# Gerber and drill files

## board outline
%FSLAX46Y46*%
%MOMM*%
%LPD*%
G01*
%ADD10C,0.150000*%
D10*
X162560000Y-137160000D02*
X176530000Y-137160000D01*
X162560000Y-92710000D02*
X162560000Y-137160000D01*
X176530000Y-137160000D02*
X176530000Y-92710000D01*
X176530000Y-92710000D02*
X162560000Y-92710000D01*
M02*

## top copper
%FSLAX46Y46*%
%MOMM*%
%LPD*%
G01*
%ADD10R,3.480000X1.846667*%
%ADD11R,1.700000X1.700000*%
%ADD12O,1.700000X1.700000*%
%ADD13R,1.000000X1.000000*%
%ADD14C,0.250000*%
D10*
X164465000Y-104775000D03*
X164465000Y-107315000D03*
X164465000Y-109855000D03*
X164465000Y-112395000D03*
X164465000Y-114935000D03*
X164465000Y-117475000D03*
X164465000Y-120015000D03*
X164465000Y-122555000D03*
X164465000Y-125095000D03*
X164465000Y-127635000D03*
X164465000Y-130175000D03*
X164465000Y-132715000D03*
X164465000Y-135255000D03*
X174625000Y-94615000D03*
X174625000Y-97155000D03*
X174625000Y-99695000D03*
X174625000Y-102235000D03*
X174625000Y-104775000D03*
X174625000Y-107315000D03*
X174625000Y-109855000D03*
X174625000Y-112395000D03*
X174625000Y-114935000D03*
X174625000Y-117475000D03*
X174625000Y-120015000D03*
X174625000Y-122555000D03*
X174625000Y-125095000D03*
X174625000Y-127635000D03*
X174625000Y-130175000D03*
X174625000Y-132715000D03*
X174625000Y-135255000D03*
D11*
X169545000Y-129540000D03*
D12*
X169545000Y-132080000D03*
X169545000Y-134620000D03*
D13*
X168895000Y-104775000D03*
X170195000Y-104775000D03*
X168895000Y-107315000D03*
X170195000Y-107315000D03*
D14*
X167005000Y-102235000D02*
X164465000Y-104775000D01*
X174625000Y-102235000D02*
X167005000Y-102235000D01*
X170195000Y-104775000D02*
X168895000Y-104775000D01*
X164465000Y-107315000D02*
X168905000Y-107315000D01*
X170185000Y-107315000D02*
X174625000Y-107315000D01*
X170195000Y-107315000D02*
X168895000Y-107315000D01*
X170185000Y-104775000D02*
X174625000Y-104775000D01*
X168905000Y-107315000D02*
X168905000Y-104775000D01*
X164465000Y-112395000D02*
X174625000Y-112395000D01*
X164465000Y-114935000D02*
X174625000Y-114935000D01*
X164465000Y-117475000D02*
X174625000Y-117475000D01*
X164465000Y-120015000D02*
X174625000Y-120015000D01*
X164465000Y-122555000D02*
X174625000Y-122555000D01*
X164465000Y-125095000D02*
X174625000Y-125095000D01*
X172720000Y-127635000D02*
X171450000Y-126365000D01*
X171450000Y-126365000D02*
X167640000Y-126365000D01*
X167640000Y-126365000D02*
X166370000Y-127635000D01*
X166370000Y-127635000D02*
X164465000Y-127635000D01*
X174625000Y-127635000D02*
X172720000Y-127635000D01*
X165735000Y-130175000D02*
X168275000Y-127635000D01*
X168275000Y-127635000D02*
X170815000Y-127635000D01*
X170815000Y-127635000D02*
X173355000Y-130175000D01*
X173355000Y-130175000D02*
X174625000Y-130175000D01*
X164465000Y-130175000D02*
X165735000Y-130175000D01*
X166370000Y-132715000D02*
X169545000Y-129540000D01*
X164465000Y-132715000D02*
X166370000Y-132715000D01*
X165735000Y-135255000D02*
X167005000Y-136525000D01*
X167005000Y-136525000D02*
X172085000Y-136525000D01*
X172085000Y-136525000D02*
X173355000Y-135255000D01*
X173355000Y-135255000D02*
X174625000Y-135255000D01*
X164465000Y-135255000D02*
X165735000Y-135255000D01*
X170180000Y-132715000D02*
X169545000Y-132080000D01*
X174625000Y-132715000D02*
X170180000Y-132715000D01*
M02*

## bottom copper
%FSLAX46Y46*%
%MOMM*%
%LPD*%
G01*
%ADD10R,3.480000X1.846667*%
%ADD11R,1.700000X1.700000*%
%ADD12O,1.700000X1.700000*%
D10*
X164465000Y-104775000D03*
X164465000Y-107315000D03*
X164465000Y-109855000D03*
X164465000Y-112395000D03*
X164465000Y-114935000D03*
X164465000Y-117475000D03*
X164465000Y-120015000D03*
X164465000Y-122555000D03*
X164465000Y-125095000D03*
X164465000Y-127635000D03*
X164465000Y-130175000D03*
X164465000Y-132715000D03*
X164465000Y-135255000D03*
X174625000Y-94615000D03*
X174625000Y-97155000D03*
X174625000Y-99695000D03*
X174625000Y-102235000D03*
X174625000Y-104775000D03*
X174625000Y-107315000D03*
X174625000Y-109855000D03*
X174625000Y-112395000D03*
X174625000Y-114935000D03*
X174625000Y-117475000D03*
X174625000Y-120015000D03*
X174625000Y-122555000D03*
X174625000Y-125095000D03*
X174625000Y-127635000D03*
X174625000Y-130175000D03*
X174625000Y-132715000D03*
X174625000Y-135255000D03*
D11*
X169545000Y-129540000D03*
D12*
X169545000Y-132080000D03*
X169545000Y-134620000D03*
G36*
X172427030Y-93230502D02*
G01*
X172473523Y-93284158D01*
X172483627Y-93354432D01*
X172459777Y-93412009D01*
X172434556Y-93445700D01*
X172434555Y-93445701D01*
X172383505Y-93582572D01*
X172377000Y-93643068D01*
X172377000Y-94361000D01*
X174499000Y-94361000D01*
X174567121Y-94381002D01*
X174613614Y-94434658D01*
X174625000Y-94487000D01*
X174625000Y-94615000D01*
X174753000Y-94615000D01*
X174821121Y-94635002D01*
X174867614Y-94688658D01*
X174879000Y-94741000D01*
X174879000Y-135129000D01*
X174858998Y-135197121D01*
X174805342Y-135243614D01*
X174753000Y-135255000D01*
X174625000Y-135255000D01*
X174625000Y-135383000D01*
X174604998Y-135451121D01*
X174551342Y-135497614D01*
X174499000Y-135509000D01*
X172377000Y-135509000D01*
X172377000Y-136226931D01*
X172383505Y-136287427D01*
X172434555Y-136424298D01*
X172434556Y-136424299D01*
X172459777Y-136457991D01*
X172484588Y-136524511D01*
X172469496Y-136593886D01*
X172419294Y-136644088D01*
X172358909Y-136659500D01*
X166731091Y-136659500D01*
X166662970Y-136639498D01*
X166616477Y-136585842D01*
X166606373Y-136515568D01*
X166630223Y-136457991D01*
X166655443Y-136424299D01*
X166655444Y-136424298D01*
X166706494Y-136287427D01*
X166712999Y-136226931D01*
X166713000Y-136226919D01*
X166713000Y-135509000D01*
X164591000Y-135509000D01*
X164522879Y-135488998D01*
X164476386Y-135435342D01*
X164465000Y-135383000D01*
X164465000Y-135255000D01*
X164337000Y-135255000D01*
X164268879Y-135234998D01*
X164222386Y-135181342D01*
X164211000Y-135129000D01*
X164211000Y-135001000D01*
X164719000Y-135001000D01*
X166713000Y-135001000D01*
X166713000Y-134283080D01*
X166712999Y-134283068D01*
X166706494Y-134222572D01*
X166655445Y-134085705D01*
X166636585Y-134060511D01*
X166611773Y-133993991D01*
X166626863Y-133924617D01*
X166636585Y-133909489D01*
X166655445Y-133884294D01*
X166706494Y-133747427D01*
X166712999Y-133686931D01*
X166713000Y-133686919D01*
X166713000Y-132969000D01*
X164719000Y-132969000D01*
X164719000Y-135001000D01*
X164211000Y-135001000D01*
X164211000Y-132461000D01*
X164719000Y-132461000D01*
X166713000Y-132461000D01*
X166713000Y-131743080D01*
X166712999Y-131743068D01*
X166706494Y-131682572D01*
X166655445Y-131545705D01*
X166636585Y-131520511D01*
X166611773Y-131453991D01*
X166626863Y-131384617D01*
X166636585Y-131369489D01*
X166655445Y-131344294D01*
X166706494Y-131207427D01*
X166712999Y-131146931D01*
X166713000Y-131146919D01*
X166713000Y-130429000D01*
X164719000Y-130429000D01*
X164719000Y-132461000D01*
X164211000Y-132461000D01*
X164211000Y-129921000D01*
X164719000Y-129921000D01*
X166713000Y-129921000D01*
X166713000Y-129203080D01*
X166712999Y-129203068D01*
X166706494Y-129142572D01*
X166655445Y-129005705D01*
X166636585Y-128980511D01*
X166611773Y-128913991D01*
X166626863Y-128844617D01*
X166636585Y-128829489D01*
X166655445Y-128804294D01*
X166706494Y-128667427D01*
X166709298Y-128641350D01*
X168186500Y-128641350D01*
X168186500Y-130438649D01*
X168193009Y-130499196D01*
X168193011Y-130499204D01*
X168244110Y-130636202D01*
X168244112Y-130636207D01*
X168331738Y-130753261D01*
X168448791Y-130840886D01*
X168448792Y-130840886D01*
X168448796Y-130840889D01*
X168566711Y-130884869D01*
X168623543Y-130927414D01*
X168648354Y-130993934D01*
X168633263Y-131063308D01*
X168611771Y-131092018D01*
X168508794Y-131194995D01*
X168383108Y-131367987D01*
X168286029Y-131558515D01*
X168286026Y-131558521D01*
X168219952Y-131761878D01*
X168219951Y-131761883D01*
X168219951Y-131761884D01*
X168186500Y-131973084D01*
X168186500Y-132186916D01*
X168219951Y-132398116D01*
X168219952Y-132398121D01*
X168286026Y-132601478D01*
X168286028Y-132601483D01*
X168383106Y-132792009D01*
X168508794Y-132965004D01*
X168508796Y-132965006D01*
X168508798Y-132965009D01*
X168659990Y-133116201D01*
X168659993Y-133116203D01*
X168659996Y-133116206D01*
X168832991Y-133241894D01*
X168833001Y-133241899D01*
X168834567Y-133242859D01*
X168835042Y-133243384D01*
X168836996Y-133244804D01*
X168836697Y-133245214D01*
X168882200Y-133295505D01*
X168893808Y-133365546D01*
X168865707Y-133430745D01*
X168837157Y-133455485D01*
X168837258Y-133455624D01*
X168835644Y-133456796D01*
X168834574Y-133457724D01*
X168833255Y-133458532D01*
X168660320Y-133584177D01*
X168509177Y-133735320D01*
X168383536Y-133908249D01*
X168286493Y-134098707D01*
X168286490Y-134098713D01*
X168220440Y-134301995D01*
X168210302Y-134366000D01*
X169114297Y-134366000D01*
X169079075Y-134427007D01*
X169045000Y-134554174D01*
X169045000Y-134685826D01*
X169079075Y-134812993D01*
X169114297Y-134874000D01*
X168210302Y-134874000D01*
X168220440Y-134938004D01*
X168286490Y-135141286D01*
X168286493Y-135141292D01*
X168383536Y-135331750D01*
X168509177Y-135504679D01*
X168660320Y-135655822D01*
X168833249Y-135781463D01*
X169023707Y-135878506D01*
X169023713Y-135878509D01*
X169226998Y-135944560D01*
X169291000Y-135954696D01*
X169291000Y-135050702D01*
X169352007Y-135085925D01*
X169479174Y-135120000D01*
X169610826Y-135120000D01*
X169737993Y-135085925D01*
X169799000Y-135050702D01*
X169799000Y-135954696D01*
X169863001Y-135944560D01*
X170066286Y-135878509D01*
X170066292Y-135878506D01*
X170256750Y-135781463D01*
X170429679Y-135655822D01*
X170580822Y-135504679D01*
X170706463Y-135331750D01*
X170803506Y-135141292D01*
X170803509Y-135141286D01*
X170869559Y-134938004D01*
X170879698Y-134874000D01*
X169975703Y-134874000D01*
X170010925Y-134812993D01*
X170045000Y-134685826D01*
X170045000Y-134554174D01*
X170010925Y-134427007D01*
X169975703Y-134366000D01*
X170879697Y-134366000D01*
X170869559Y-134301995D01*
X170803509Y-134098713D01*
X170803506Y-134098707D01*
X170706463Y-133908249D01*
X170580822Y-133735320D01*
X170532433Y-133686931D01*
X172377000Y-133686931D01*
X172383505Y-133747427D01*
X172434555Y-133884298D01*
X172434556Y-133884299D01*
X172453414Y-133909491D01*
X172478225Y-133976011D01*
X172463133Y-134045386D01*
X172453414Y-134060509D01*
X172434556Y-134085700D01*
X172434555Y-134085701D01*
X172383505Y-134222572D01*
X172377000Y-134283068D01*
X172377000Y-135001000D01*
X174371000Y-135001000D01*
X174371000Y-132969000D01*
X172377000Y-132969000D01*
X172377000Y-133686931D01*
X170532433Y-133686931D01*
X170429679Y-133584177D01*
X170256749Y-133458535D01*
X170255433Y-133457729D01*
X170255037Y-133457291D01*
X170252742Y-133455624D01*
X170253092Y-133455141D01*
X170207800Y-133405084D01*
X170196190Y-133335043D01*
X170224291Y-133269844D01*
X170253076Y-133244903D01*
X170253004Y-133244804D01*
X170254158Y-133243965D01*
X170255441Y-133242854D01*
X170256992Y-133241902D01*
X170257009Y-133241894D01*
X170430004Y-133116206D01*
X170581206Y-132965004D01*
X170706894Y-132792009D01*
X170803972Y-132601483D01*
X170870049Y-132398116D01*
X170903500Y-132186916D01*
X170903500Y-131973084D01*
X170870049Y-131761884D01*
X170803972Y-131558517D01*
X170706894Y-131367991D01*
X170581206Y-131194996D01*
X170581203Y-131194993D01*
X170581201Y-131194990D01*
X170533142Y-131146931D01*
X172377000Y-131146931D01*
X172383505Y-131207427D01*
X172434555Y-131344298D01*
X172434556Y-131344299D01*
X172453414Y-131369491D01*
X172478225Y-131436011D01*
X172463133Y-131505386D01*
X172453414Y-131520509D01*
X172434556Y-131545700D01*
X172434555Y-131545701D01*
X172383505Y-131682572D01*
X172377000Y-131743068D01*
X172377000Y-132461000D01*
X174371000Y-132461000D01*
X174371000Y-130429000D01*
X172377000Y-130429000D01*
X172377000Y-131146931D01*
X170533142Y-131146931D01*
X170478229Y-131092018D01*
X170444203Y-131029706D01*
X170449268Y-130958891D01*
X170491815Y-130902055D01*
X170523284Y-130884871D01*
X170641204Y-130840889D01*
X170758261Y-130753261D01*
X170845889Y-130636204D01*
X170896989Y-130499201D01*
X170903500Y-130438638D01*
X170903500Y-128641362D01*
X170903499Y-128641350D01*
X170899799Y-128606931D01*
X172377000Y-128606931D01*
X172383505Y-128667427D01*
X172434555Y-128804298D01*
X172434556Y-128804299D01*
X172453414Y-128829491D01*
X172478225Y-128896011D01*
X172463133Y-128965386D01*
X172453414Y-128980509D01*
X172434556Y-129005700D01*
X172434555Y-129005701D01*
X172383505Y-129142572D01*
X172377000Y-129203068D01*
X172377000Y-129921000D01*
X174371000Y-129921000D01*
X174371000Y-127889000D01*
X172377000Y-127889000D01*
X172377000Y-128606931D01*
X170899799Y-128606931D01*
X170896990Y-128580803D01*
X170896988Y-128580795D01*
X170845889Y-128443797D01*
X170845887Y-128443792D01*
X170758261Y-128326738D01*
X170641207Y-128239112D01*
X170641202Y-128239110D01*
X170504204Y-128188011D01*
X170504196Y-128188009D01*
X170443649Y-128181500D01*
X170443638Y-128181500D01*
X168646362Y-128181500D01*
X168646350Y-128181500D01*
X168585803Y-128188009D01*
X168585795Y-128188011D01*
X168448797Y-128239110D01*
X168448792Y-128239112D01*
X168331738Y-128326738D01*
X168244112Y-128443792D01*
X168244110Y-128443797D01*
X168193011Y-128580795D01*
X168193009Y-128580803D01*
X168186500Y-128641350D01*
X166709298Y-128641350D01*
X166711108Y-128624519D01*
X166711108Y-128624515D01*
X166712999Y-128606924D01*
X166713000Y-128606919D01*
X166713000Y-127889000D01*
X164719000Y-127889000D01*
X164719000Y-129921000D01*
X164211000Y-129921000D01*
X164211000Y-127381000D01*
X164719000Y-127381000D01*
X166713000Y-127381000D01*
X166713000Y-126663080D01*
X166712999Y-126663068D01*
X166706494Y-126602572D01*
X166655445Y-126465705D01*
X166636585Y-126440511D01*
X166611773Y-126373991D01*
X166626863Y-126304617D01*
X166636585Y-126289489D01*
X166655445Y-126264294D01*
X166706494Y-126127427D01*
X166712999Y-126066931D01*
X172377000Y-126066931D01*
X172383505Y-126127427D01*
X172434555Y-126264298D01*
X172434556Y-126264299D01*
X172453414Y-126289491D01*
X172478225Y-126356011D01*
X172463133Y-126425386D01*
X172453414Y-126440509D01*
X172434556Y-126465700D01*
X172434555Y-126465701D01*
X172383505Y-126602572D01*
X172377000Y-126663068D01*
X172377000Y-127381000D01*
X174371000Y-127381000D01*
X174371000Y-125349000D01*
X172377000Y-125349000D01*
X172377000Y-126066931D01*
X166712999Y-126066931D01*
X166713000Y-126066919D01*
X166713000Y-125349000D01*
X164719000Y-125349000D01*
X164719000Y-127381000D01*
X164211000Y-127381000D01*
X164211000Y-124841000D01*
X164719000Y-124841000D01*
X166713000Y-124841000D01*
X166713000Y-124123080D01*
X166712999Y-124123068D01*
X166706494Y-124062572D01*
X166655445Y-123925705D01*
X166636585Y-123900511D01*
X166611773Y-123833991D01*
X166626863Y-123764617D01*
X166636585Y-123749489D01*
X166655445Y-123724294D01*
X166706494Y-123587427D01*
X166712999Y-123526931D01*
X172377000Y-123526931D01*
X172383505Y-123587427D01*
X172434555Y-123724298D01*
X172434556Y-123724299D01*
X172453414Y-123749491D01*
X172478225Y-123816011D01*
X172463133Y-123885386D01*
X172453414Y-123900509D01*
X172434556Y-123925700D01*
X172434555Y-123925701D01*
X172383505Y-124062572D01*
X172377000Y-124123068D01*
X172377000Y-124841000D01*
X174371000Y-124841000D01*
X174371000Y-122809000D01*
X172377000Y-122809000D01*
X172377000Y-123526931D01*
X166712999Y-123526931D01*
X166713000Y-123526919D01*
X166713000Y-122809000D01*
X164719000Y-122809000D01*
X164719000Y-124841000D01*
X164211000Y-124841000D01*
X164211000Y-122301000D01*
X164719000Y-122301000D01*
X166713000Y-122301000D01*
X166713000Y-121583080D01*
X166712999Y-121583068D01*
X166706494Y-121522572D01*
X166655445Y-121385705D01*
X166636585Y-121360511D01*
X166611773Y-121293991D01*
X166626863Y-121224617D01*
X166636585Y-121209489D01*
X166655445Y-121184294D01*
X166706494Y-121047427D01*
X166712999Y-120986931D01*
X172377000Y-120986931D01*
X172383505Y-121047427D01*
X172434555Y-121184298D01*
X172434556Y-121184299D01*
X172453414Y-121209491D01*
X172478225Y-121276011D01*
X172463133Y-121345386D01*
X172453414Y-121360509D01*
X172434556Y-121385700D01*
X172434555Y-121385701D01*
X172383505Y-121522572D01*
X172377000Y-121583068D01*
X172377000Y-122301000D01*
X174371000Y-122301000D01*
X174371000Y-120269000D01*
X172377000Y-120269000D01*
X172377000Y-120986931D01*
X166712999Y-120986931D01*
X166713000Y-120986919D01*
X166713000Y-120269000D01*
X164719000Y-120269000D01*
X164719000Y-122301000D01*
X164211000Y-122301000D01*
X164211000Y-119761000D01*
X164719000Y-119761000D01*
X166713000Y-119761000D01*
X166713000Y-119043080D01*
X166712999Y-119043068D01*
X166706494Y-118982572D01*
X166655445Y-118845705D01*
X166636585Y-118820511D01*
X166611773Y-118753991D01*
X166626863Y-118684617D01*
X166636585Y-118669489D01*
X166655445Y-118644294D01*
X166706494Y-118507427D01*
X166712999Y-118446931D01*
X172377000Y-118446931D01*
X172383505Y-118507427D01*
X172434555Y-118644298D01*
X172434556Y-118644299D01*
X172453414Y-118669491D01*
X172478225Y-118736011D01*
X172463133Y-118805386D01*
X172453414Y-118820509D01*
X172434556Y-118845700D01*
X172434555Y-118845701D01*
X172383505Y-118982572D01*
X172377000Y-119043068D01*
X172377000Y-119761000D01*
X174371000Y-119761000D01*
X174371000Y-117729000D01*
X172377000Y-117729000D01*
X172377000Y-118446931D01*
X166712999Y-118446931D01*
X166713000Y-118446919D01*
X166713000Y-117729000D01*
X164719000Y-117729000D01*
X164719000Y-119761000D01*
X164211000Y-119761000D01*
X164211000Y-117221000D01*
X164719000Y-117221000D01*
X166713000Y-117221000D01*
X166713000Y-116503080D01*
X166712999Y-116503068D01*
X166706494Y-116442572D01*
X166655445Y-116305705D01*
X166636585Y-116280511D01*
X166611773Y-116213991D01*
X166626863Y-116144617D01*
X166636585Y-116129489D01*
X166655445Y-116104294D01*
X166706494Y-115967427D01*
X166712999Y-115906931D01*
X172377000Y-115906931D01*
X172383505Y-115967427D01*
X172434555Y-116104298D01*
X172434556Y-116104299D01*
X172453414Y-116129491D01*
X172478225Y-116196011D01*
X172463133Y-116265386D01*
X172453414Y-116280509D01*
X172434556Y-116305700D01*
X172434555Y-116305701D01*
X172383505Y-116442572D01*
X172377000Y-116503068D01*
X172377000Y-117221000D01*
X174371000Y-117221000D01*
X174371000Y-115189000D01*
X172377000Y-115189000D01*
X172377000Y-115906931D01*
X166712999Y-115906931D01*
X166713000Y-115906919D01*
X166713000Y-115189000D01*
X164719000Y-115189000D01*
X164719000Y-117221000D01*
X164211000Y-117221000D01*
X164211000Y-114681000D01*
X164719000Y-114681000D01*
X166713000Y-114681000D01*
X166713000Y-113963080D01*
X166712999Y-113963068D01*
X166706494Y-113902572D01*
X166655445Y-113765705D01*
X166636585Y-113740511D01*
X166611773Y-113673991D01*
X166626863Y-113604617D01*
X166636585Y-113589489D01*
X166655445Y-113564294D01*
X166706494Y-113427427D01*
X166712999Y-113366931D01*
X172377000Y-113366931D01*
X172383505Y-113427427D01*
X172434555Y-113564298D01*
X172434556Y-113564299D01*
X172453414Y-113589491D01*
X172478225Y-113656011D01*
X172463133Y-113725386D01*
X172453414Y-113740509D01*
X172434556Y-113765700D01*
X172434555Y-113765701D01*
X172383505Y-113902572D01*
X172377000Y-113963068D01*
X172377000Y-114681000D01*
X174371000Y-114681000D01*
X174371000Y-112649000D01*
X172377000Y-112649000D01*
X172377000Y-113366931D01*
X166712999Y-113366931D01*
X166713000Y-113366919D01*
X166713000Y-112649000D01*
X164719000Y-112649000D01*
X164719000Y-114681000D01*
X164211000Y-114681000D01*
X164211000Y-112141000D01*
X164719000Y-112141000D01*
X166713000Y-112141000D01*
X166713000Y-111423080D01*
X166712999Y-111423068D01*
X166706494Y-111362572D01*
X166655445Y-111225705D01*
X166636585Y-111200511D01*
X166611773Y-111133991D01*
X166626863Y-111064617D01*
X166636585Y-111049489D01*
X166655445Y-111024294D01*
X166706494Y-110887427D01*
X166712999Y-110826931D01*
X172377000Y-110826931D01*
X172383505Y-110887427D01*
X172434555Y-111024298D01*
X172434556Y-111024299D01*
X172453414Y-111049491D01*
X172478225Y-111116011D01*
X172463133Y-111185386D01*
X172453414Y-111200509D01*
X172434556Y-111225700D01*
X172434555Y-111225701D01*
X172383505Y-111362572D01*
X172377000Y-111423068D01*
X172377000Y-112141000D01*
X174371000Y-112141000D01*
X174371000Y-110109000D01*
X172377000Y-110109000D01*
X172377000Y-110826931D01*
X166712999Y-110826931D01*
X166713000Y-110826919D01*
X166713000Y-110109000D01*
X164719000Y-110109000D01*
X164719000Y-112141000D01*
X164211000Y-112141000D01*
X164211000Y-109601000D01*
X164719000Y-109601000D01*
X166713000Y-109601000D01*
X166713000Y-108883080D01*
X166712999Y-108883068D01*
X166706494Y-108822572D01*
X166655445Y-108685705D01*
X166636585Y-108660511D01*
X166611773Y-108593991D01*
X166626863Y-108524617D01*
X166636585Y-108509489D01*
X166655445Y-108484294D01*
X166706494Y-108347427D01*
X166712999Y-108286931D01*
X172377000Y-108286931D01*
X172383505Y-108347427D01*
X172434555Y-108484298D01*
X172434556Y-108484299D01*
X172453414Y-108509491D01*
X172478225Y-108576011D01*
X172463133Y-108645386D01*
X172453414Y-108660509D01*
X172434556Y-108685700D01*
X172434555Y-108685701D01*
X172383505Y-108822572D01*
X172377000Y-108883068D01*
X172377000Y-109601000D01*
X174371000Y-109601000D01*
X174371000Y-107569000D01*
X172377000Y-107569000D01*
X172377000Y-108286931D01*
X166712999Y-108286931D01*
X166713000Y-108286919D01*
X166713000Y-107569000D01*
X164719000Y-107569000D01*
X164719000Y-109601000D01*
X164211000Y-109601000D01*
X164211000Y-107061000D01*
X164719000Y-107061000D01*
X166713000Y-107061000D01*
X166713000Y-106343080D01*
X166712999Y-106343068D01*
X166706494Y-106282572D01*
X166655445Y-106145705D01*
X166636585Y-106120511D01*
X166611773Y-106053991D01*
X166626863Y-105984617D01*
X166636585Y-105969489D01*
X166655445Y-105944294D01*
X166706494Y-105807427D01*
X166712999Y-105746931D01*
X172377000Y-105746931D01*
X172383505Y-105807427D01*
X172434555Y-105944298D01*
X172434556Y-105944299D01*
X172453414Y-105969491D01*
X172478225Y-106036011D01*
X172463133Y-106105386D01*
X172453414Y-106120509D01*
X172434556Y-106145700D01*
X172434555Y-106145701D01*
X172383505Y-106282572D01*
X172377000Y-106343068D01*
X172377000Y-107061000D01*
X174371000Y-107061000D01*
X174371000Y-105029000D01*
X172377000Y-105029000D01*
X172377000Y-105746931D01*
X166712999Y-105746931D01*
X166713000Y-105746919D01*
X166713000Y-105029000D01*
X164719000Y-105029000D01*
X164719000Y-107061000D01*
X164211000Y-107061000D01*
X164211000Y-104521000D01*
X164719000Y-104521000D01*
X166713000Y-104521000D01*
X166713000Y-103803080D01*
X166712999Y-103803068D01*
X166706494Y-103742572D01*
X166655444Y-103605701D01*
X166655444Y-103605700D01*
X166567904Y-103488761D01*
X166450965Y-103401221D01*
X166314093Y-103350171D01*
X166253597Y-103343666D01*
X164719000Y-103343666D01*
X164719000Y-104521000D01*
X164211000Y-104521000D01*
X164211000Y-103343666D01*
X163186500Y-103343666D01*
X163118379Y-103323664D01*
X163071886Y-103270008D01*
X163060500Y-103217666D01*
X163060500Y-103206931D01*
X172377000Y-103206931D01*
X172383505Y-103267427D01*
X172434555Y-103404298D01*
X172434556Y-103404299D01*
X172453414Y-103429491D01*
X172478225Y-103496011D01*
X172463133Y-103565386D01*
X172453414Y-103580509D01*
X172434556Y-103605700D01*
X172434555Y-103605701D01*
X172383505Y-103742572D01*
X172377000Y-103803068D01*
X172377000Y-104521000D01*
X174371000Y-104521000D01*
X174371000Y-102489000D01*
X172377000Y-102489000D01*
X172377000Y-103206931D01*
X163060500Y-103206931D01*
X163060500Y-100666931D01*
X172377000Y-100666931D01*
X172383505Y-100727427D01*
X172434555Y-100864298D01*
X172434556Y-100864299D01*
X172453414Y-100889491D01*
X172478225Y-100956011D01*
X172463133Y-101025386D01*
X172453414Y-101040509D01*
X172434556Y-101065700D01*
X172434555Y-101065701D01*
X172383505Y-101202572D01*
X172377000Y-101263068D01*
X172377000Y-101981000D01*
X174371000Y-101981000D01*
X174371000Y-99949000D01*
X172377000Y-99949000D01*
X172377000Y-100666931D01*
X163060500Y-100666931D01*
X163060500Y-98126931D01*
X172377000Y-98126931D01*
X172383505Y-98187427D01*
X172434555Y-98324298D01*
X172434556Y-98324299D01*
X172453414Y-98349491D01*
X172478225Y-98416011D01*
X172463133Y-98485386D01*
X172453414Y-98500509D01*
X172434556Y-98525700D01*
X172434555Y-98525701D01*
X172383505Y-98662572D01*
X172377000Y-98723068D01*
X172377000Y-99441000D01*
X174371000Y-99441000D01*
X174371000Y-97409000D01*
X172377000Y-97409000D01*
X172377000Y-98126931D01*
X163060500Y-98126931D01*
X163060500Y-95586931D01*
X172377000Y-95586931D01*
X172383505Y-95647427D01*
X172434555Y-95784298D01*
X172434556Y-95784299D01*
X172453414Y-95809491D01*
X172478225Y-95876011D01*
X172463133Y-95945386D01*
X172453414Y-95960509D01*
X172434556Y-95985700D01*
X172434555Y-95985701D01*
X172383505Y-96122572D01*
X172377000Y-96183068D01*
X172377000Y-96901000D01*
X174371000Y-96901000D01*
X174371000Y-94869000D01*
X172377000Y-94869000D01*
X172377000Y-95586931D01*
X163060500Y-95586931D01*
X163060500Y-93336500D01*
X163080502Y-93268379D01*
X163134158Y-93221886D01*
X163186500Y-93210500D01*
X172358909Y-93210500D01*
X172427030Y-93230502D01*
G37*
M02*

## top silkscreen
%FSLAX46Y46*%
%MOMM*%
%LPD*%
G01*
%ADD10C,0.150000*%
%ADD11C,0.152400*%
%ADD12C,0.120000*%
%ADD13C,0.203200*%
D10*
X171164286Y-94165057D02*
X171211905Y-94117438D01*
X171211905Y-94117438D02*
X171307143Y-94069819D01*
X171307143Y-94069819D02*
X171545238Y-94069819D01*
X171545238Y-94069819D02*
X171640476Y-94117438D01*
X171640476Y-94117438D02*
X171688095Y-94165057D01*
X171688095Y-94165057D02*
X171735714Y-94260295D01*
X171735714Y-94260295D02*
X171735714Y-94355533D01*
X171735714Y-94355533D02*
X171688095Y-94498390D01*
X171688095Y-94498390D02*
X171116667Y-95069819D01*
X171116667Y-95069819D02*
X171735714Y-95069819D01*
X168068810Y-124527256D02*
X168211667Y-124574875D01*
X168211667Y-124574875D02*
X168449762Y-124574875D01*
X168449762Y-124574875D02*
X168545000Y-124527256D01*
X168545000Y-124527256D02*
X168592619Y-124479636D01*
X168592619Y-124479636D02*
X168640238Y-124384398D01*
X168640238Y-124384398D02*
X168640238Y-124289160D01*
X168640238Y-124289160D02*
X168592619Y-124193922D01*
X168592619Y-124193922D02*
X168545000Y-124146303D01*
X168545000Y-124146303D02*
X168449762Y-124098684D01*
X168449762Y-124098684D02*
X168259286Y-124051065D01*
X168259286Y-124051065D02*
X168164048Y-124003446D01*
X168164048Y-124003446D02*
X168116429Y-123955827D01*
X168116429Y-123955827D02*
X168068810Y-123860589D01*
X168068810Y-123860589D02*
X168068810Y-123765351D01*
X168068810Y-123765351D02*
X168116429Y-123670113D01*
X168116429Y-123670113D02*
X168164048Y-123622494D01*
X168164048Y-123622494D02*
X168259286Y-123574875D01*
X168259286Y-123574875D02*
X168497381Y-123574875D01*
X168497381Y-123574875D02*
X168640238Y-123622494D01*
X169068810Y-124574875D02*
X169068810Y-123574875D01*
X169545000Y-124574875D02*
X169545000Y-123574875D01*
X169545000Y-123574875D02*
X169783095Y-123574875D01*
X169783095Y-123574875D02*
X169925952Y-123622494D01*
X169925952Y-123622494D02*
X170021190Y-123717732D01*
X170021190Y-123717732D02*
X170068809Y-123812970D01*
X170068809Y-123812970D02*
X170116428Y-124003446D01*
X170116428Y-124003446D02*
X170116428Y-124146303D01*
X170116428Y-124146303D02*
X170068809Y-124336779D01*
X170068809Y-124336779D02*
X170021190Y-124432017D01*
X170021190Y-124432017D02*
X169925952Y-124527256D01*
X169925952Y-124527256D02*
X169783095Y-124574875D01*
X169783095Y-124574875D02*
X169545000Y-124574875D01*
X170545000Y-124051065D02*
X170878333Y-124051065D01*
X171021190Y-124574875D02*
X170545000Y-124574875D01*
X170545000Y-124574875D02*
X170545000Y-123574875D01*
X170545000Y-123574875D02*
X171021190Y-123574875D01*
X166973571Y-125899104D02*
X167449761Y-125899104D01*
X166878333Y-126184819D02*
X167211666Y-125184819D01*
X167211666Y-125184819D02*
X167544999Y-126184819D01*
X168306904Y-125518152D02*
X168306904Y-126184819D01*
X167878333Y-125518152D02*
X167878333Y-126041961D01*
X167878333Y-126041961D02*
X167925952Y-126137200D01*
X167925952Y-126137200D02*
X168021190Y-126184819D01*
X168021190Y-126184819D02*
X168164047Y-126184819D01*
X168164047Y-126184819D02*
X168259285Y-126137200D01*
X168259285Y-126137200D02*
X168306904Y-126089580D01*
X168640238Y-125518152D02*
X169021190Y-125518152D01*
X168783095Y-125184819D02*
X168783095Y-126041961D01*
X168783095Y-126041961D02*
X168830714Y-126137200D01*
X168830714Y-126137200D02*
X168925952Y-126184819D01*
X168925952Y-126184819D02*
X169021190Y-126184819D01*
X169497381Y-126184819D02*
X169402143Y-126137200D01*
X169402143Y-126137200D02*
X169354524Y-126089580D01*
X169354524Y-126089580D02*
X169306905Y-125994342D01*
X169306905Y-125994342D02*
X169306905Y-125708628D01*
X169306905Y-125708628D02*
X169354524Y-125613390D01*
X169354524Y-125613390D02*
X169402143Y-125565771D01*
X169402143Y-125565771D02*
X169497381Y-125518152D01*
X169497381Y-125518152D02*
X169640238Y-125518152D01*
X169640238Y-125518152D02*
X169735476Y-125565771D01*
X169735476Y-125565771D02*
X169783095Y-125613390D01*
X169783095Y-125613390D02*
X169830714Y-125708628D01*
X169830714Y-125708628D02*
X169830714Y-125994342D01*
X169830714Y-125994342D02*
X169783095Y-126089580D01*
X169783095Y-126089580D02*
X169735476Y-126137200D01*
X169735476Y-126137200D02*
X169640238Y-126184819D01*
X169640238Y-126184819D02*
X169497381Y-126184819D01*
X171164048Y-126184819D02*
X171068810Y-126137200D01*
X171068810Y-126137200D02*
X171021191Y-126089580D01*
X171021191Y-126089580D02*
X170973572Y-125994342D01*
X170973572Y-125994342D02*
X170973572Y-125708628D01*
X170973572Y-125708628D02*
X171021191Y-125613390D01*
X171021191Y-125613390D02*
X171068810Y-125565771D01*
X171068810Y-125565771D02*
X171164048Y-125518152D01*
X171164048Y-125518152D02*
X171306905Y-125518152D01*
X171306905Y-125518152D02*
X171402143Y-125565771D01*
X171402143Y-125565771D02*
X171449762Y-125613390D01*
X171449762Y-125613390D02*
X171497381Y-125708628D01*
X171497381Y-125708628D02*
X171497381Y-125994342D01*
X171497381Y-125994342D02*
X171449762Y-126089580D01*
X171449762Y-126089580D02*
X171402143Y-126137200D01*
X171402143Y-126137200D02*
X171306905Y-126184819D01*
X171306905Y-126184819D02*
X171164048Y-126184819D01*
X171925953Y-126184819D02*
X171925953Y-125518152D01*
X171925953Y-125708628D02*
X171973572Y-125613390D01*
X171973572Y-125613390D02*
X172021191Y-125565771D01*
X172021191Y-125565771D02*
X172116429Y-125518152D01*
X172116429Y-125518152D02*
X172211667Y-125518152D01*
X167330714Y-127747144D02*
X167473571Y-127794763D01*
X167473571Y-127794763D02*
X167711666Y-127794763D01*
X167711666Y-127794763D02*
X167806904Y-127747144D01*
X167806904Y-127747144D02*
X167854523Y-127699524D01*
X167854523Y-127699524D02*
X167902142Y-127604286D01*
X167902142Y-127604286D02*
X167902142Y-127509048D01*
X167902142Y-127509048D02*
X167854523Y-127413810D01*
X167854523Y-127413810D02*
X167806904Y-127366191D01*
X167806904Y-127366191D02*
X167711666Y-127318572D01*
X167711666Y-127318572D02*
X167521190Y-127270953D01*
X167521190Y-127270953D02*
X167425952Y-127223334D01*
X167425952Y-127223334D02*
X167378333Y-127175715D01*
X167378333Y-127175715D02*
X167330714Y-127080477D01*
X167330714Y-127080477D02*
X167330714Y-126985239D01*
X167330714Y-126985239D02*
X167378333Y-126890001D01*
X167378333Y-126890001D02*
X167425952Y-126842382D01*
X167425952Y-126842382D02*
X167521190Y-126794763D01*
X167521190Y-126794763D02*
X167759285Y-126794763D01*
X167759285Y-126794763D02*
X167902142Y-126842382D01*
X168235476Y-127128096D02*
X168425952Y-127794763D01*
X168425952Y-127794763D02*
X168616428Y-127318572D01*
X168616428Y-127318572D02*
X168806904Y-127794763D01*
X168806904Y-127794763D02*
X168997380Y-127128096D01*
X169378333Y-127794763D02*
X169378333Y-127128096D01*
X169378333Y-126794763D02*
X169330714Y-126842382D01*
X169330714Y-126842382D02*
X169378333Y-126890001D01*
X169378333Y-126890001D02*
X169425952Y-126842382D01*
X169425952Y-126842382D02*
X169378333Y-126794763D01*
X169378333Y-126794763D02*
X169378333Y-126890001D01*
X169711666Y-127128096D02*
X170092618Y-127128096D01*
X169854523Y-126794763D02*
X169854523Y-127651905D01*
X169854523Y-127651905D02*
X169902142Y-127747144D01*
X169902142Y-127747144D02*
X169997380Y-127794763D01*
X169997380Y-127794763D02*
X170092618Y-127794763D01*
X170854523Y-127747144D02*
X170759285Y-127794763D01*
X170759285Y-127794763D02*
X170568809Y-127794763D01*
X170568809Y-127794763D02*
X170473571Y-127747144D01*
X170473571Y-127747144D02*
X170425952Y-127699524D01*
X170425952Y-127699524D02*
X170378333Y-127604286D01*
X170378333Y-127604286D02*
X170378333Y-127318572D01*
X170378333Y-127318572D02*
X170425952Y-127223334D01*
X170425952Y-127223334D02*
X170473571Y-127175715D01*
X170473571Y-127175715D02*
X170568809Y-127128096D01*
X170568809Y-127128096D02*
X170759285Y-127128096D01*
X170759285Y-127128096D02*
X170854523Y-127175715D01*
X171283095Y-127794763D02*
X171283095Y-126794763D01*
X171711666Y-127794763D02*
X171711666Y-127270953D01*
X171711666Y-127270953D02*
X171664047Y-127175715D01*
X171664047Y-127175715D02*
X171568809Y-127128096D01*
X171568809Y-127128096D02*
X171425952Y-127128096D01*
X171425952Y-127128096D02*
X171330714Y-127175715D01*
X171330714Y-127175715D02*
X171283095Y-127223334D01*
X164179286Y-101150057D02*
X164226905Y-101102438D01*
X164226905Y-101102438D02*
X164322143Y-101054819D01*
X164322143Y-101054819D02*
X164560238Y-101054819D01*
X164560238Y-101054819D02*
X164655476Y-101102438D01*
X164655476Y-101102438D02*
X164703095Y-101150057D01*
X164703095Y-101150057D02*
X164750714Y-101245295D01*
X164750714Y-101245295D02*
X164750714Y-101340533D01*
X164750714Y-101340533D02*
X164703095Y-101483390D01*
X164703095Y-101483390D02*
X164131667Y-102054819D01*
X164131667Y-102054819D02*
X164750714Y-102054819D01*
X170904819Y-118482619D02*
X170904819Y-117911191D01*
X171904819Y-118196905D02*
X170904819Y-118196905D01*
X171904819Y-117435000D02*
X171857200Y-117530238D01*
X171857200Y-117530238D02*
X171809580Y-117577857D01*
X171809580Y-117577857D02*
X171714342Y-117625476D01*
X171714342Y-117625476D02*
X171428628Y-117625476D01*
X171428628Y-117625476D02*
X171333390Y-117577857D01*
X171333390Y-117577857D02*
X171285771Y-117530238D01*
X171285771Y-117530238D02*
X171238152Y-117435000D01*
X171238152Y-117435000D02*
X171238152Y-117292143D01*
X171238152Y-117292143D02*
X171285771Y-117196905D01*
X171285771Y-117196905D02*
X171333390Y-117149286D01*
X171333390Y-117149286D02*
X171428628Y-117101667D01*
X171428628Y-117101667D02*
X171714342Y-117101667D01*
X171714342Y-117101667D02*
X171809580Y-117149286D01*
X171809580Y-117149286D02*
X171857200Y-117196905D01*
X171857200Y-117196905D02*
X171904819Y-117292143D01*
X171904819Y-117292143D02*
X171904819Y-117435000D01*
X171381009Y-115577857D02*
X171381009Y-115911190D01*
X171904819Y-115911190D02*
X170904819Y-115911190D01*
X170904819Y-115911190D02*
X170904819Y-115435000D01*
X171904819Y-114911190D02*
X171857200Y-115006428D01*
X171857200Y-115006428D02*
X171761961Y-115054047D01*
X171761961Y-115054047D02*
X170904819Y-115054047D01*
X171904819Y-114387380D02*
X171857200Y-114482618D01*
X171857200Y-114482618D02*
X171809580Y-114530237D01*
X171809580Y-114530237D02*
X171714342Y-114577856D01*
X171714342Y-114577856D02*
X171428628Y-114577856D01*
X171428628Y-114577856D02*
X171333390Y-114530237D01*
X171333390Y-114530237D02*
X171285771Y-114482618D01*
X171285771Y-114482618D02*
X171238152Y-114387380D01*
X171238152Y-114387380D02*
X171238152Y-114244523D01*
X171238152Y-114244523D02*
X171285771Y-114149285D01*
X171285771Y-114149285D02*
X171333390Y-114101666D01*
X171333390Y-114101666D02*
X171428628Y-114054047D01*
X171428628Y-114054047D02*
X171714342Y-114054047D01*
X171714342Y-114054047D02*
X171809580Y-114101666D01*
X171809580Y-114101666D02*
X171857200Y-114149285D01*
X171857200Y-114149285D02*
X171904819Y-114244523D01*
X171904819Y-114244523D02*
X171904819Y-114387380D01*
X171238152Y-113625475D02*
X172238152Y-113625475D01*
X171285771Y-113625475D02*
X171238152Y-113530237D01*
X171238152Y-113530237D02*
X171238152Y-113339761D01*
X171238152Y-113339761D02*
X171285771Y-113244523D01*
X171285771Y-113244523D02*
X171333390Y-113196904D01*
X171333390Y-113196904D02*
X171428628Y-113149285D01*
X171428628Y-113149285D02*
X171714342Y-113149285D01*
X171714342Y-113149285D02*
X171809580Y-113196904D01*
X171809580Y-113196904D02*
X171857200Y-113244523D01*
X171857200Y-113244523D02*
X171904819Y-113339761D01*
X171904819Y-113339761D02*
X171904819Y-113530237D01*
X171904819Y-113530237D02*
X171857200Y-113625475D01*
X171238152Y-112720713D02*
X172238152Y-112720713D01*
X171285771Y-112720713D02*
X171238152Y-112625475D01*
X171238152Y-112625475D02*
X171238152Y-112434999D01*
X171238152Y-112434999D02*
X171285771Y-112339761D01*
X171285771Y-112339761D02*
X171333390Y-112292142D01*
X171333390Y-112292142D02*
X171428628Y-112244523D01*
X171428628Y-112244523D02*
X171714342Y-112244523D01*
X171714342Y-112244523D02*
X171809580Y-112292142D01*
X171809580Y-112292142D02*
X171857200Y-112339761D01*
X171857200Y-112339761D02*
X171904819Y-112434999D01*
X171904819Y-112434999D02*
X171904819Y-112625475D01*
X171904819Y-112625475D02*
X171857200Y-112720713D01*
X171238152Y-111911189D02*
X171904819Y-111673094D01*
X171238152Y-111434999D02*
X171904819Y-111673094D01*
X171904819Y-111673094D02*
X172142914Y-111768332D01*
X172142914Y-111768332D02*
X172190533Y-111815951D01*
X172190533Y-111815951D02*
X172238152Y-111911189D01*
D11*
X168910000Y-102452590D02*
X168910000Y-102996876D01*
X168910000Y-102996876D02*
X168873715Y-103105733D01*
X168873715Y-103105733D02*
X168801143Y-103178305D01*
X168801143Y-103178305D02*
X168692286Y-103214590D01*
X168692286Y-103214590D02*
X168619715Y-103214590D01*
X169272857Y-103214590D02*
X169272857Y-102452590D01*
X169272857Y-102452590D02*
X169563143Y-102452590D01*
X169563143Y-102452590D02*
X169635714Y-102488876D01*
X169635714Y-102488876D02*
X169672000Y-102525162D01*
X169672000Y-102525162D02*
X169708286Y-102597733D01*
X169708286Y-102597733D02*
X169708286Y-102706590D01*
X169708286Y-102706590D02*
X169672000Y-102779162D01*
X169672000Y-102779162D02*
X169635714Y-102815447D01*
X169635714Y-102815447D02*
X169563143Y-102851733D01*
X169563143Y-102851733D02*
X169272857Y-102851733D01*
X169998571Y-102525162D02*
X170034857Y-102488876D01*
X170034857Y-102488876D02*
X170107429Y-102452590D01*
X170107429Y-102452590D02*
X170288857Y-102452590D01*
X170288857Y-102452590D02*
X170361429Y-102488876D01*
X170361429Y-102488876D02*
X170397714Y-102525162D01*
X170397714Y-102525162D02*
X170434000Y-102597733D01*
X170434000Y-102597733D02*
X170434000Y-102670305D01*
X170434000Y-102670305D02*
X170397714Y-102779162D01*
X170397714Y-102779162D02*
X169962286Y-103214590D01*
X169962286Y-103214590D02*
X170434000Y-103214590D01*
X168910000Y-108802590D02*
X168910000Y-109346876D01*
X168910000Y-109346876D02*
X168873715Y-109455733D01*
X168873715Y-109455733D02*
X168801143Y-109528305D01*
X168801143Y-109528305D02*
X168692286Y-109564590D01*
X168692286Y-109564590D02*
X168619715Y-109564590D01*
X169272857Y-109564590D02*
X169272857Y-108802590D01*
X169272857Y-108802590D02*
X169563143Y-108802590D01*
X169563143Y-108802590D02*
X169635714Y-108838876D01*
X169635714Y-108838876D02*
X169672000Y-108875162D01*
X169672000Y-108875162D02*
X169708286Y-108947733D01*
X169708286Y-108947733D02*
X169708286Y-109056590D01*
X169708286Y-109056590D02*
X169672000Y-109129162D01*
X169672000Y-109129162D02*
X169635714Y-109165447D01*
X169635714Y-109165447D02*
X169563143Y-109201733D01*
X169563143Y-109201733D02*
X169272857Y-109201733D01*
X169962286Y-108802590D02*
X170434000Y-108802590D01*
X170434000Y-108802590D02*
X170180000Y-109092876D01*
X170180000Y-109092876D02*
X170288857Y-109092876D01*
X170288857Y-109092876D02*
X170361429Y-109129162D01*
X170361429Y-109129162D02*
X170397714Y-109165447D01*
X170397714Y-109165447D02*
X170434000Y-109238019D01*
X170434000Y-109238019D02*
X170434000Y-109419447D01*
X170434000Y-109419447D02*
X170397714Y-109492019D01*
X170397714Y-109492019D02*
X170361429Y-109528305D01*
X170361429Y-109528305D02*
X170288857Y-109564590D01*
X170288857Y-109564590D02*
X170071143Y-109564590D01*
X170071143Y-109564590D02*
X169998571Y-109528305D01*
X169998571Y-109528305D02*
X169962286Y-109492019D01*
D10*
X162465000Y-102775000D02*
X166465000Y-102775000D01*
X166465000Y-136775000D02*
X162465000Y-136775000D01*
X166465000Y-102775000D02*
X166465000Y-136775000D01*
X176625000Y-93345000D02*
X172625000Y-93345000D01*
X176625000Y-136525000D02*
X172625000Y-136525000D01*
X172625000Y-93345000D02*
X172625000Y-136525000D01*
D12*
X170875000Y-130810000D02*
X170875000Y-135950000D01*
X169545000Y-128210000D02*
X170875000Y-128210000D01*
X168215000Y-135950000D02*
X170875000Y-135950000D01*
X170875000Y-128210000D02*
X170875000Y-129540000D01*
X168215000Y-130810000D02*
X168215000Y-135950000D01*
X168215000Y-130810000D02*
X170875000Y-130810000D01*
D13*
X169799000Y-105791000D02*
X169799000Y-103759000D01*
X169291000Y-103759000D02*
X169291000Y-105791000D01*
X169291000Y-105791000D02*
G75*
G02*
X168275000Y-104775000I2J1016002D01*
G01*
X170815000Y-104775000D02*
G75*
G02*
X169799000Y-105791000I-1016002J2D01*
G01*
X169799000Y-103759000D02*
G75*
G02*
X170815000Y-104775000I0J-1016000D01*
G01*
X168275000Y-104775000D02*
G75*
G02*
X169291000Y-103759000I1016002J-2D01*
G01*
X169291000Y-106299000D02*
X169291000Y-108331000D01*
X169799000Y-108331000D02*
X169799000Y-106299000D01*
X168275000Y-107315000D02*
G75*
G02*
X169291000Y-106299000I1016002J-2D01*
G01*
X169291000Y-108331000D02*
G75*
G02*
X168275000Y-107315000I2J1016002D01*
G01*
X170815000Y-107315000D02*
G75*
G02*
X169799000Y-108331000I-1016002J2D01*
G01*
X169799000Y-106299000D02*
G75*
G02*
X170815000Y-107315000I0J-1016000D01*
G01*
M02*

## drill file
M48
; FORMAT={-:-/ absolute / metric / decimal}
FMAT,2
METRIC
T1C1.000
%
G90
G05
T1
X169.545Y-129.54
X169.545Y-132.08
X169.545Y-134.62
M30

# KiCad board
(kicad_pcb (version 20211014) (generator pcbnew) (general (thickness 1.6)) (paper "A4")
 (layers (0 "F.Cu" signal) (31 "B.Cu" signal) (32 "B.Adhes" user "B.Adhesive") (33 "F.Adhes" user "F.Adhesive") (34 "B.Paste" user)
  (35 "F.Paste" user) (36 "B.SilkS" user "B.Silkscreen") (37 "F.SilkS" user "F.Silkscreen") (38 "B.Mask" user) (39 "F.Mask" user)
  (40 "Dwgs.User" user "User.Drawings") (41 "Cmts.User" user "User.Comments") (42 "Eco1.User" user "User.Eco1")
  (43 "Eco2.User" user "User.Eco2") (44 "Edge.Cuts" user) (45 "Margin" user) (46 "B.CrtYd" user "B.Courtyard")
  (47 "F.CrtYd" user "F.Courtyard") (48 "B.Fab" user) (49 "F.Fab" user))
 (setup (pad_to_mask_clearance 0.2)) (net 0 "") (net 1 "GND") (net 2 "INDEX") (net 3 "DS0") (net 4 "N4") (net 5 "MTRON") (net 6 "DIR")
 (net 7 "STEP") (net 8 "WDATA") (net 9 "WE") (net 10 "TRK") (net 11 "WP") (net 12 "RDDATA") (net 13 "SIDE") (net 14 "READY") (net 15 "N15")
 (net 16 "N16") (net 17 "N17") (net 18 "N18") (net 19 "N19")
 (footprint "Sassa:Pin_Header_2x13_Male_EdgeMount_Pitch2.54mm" (layer "F.Cu") (at 164.465 104.775 -90)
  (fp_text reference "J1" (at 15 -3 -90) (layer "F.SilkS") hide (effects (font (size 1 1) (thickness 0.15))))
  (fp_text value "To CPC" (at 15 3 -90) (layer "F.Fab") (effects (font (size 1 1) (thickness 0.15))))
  (fp_line (start -2 2) (end -2 -2) (layer "F.SilkS") (width 0.15))
  (fp_line (start 32 -2) (end 32 2) (layer "F.SilkS") (width 0.15))
  (fp_line (start -2 -2) (end 32 -2) (layer "F.SilkS") (width 0.15))
  (pad "1" smd rect locked (at 0 0 270) (size 1.846667 3.48) (layers "B.Cu" "B.Paste" "B.Mask") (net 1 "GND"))
  (pad "2" smd rect locked (at 0 0 270) (size 1.846667 3.48) (layers "F.Cu" "F.Paste" "F.Mask") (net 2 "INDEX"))
  (pad "3" smd rect locked (at 2.54 0 270) (size 1.846667 3.48) (layers "B.Cu" "B.Paste" "B.Mask") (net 1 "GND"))
  (pad "4" smd rect locked (at 2.54 0 270) (size 1.846667 3.48) (layers "F.Cu" "F.Paste" "F.Mask") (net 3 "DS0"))
  (pad "5" smd rect locked (at 5.08 0 270) (size 1.846667 3.48) (layers "B.Cu" "B.Paste" "B.Mask") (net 1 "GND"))
  (pad "6" smd rect locked (at 5.08 0 270) (size 1.846667 3.48) (layers "F.Cu" "F.Paste" "F.Mask") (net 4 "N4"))
  (pad "7" smd rect locked (at 7.62 0 270) (size 1.846667 3.48) (layers "B.Cu" "B.Paste" "B.Mask") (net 1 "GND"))
  (pad "8" smd rect locked (at 7.62 0 270) (size 1.846667 3.48) (layers "F.Cu" "F.Paste" "F.Mask") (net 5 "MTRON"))
  (pad "9" smd rect locked (at 10.16 0 270) (size 1.846667 3.48) (layers "B.Cu" "B.Paste" "B.Mask") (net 1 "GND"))
  (pad "10" smd rect locked (at 10.16 0 270) (size 1.846667 3.48) (layers "F.Cu" "F.Paste" "F.Mask") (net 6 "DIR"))
  (pad "11" smd rect locked (at 12.7 0 270) (size 1.846667 3.48) (layers "B.Cu" "B.Paste" "B.Mask") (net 1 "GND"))
  (pad "12" smd rect locked (at 12.7 0 270) (size 1.846667 3.48) (layers "F.Cu" "F.Paste" "F.Mask") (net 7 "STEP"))
  (pad "13" smd rect locked (at 15.24 0 270) (size 1.846667 3.48) (layers "B.Cu" "B.Paste" "B.Mask") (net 1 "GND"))
  (pad "14" smd rect locked (at 15.24 0 270) (size 1.846667 3.48) (layers "F.Cu" "F.Paste" "F.Mask") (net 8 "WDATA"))
  (pad "15" smd rect locked (at 17.78 0 270) (size 1.846667 3.48) (layers "B.Cu" "B.Paste" "B.Mask") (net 1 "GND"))
  (pad "16" smd rect locked (at 17.78 0 270) (size 1.846667 3.48) (layers "F.Cu" "F.Paste" "F.Mask") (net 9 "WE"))
  (pad "17" smd rect locked (at 20.32 0 270) (size 1.846667 3.48) (layers "B.Cu" "B.Paste" "B.Mask") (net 1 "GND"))
  (pad "18" smd rect locked (at 20.32 0 270) (size 1.846667 3.48) (layers "F.Cu" "F.Paste" "F.Mask") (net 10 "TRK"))
  (pad "19" smd rect locked (at 22.86 0 270) (size 1.846667 3.48) (layers "B.Cu" "B.Paste" "B.Mask") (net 1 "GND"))
  (pad "20" smd rect locked (at 22.86 0 270) (size 1.846667 3.48) (layers "F.Cu" "F.Paste" "F.Mask") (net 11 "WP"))
  (pad "21" smd rect locked (at 25.4 0 270) (size 1.846667 3.48) (layers "B.Cu" "B.Paste" "B.Mask") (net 1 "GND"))
  (pad "22" smd rect locked (at 25.4 0 270) (size 1.846667 3.48) (layers "F.Cu" "F.Paste" "F.Mask") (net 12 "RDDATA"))
  (pad "23" smd rect locked (at 27.94 0 270) (size 1.846667 3.48) (layers "B.Cu" "B.Paste" "B.Mask") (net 1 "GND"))
  (pad "24" smd rect locked (at 27.94 0 270) (size 1.846667 3.48) (layers "F.Cu" "F.Paste" "F.Mask") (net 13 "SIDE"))
  (pad "25" smd rect locked (at 30.48 0 270) (size 1.846667 3.48) (layers "B.Cu" "B.Paste" "B.Mask") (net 1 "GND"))
  (pad "26" smd rect locked (at 30.48 0 270) (size 1.846667 3.48) (layers "F.Cu" "F.Paste" "F.Mask") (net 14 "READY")))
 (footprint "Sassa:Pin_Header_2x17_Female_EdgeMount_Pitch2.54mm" (layer "F.Cu") (at 174.625 135.255 90)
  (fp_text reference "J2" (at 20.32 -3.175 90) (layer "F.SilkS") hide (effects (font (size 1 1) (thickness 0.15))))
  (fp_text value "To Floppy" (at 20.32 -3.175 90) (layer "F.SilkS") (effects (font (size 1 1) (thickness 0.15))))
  (fp_line (start 41.91 2) (end 41.91 -2) (layer "F.SilkS") (width 0.15))
  (fp_line (start -1.27 2) (end -1.27 -2) (layer "F.SilkS") (width 0.15))
  (fp_line (start 41.91 -2) (end -1.27 -2) (layer "F.SilkS") (width 0.15))
  (pad "1" smd rect (at 40.64 0 90) (size 1.846667 3.48) (layers "B.Cu" "B.Paste" "B.Mask") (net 1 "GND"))
  (pad "2" smd rect (at 40.64 0 90) (size 1.846667 3.48) (layers "F.Cu" "F.Paste" "F.Mask") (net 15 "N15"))
  (pad "3" smd rect (at 38.1 0 90) (size 1.846667 3.48) (layers "B.Cu" "B.Paste" "B.Mask") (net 1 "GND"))
  (pad "4" smd rect (at 38.1 0 90) (size 1.846667 3.48) (layers "F.Cu" "F.Paste" "F.Mask") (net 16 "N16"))
  (pad "5" smd rect (at 35.56 0 90) (size 1.846667 3.48) (layers "B.Cu" "B.Paste" "B.Mask") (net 1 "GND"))
  (pad "6" smd rect (at 35.56 0 90) (size 1.846667 3.48) (layers "F.Cu" "F.Paste" "F.Mask") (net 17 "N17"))
  (pad "7" smd rect (at 33.02 0 90) (size 1.846667 3.48) (layers "B.Cu" "B.Paste" "B.Mask") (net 1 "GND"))
  (pad "8" smd rect (at 33.02 0 90) (size 1.846667 3.48) (layers "F.Cu" "F.Paste" "F.Mask") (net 2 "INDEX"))
  (pad "9" smd rect (at 30.48 0 90) (size 1.846667 3.48) (layers "B.Cu" "B.Paste" "B.Mask") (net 1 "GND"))
  (pad "10" smd rect (at 30.48 0 90) (size 1.846667 3.48) (layers "F.Cu" "F.Paste" "F.Mask") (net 3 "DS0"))
  (pad "11" smd rect (at 27.94 0 90) (size 1.846667 3.48) (layers "B.Cu" "B.Paste" "B.Mask") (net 1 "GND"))
  (pad "12" smd rect (at 27.94 0 90) (size 1.846667 3.48) (layers "F.Cu" "F.Paste" "F.Mask") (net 3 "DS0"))
  (pad "13" smd rect (at 25.4 0 90) (size 1.846667 3.48) (layers "B.Cu" "B.Paste" "B.Mask") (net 1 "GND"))
  (pad "14" smd rect (at 25.4 0 90) (size 1.846667 3.48) (layers "F.Cu" "F.Paste" "F.Mask") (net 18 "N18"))
  (pad "15" smd rect (at 22.86 0 90) (size 1.846667 3.48) (layers "B.Cu" "B.Paste" "B.Mask") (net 1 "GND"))
  (pad "16" smd rect (at 22.86 0 90) (size 1.846667 3.48) (layers "F.Cu" "F.Paste" "F.Mask") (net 5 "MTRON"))
  (pad "17" smd rect (at 20.32 0 90) (size 1.846667 3.48) (layers "B.Cu" "B.Paste" "B.Mask") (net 1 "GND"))
  (pad "18" smd rect (at 20.32 0 90) (size 1.846667 3.48) (layers "F.Cu" "F.Paste" "F.Mask") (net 6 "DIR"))
  (pad "19" smd rect (at 17.78 0 90) (size 1.846667 3.48) (layers "B.Cu" "B.Paste" "B.Mask") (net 1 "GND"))
  (pad "20" smd rect (at 17.78 0 90) (size 1.846667 3.48) (layers "F.Cu" "F.Paste" "F.Mask") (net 7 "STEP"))
  (pad "21" smd rect (at 15.24 0 90) (size 1.846667 3.48) (layers "B.Cu" "B.Paste" "B.Mask") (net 1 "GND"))
  (pad "22" smd rect (at 15.24 0 90) (size 1.846667 3.48) (layers "F.Cu" "F.Paste" "F.Mask") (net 8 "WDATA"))
  (pad "23" smd rect (at 12.7 0 90) (size 1.846667 3.48) (layers "B.Cu" "B.Paste" "B.Mask") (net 1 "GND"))
  (pad "24" smd rect (at 12.7 0 90) (size 1.846667 3.48) (layers "F.Cu" "F.Paste" "F.Mask") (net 9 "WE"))
  (pad "25" smd rect (at 10.16 0 90) (size 1.846667 3.48) (layers "B.Cu" "B.Paste" "B.Mask") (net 1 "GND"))
  (pad "26" smd rect (at 10.16 0 90) (size 1.846667 3.48) (layers "F.Cu" "F.Paste" "F.Mask") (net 10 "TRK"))
  (pad "27" smd rect (at 7.62 0 90) (size 1.846667 3.48) (layers "B.Cu" "B.Paste" "B.Mask") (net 1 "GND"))
  (pad "28" smd rect (at 7.62 0 90) (size 1.846667 3.48) (layers "F.Cu" "F.Paste" "F.Mask") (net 11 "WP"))
  (pad "29" smd rect (at 5.08 0 90) (size 1.846667 3.48) (layers "B.Cu" "B.Paste" "B.Mask") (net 1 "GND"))
  (pad "30" smd rect (at 5.08 0 90) (size 1.846667 3.48) (layers "F.Cu" "F.Paste" "F.Mask") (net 12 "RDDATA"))
  (pad "31" smd rect (at 2.54 0 90) (size 1.846667 3.48) (layers "B.Cu" "B.Paste" "B.Mask") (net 1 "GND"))
  (pad "32" smd rect (at 2.54 0 90) (size 1.846667 3.48) (layers "F.Cu" "F.Paste" "F.Mask") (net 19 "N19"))
  (pad "33" smd rect (at 0 0 90) (size 1.846667 3.48) (layers "B.Cu" "B.Paste" "B.Mask") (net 1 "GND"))
  (pad "34" smd rect (at 0 0 90) (size 1.846667 3.48) (layers "F.Cu" "F.Paste" "F.Mask") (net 14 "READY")))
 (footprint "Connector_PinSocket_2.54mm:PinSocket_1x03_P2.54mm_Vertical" (layer "F.Cu") (at 169.545 129.54)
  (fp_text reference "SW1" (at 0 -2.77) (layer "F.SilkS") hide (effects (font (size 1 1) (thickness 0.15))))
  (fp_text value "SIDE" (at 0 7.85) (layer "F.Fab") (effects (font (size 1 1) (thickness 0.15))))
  (fp_line (start 1.33 1.27) (end 1.33 6.41) (layer "F.SilkS") (width 0.12))
  (fp_line (start 0 -1.33) (end 1.33 -1.33) (layer "F.SilkS") (width 0.12))
  (fp_line (start -1.33 6.41) (end 1.33 6.41) (layer "F.SilkS") (width 0.12))
  (fp_line (start 1.33 -1.33) (end 1.33 0) (layer "F.SilkS") (width 0.12))
  (fp_line (start -1.33 1.27) (end -1.33 6.41) (layer "F.SilkS") (width 0.12))
  (fp_line (start -1.33 1.27) (end 1.33 1.27) (layer "F.SilkS") (width 0.12))
  (pad "1" thru_hole rect (at 0 0) (size 1.7 1.7) (drill 1) (layers *.Cu *.Mask) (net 13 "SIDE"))
  (pad "2" thru_hole oval (at 0 2.54) (size 1.7 1.7) (drill 1) (layers *.Cu *.Mask) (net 19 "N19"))
  (pad "3" thru_hole oval (at 0 5.08) (size 1.7 1.7) (drill 1) (layers *.Cu *.Mask) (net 1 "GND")))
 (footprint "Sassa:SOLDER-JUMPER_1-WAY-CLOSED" (layer "F.Cu") (at 169.545 104.775)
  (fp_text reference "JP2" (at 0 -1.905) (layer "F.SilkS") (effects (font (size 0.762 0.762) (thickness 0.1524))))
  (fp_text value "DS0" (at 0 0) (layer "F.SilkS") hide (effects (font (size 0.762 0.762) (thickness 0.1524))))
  (fp_line (start 0.254 1.016) (end 0.254 -1.016) (layer "F.SilkS") (width 0.2032))
  (fp_line (start -0.254 -1.016) (end -0.254 1.016) (layer "F.SilkS") (width 0.2032))
  (fp_arc (start -0.254 1.016) (mid -0.97242 0.71842) (end -1.27 0) (layer "F.SilkS") (width 0.2032))
  (fp_arc (start 1.27 0) (mid 0.97242 0.71842) (end 0.254 1.016) (layer "F.SilkS") (width 0.2032))
  (fp_arc (start 0.254 -1.016) (mid 0.97242 -0.71842) (end 1.27 0) (layer "F.SilkS") (width 0.2032))
  (fp_arc (start -1.27 0) (mid -0.97242 -0.71842) (end -0.254 -1.016) (layer "F.SilkS") (width 0.2032))
  (pad "1" smd rect locked (at -0.65 0) (size 1 1) (layers "F.Cu" "F.Paste" "F.Mask") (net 3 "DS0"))
  (pad "2" smd rect locked (at 0.65 0) (size 1 1) (layers "F.Cu" "F.Paste" "F.Mask") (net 3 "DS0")))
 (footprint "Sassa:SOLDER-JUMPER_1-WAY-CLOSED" (layer "F.Cu") (at 169.545 107.315)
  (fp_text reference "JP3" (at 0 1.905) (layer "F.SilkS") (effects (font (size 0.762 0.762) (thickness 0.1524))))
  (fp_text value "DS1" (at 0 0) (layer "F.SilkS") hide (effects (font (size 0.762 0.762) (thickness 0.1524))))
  (fp_line (start -0.254 -1.016) (end -0.254 1.016) (layer "F.SilkS") (width 0.2032))
  (fp_line (start 0.254 1.016) (end 0.254 -1.016) (layer "F.SilkS") (width 0.2032))
  (fp_arc (start -1.27 0) (mid -0.97242 -0.71842) (end -0.254 -1.016) (layer "F.SilkS") (width 0.2032))
  (fp_arc (start -0.254 1.016) (mid -0.97242 0.71842) (end -1.27 0) (layer "F.SilkS") (width 0.2032))
  (fp_arc (start 1.27 0) (mid 0.97242 0.71842) (end 0.254 1.016) (layer "F.SilkS") (width 0.2032))
  (fp_arc (start 0.254 -1.016) (mid 0.97242 -0.71842) (end 1.27 0) (layer "F.SilkS") (width 0.2032))
  (pad "1" smd rect locked (at -0.65 0) (size 1 1) (layers "F.Cu" "F.Paste" "F.Mask") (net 3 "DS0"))
  (pad "2" smd rect locked (at 0.65 0) (size 1 1) (layers "F.Cu" "F.Paste" "F.Mask") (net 3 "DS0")))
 (gr_line (start 162.56 137.16) (end 176.53 137.16) (layer "Edge.Cuts") (width 0.15))
 (gr_line (start 162.56 92.71) (end 162.56 137.16) (layer "Edge.Cuts") (width 0.15))
 (gr_line (start 176.53 137.16) (end 176.53 92.71) (layer "Edge.Cuts") (width 0.15))
 (gr_line (start 176.53 92.71) (end 162.56 92.71) (layer "Edge.Cuts") (width 0.15))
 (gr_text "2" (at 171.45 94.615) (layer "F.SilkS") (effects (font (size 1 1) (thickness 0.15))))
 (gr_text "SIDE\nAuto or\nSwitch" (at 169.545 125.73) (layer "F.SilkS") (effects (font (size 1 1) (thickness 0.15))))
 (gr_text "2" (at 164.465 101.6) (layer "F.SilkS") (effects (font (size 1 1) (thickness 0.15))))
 (segment (start 167.005 102.235) (end 164.465 104.775) (width 0.25) (layer "F.Cu") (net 2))
 (segment (start 174.625 102.235) (end 167.005 102.235) (width 0.25) (layer "F.Cu") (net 2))
 (segment (start 170.195 104.775) (end 168.895 104.775) (width 0.25) (layer "F.Cu") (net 3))
 (segment (start 164.465 107.315) (end 168.905 107.315) (width 0.25) (layer "F.Cu") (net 3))
 (segment (start 170.185 107.315) (end 174.625 107.315) (width 0.25) (layer "F.Cu") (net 3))
 (segment (start 170.195 107.315) (end 168.895 107.315) (width 0.25) (layer "F.Cu") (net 3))
 (segment (start 170.185 104.775) (end 174.625 104.775) (width 0.25) (layer "F.Cu") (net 3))
 (segment (start 168.905 107.315) (end 168.905 104.775) (width 0.25) (layer "F.Cu") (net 3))
 (segment (start 164.465 112.395) (end 174.625 112.395) (width 0.25) (layer "F.Cu") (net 5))
 (segment (start 164.465 114.935) (end 174.625 114.935) (width 0.25) (layer "F.Cu") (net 6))
 (segment (start 164.465 117.475) (end 174.625 117.475) (width 0.25) (layer "F.Cu") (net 7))
 (segment (start 164.465 120.015) (end 174.625 120.015) (width 0.25) (layer "F.Cu") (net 8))
 (segment (start 164.465 122.555) (end 174.625 122.555) (width 0.25) (layer "F.Cu") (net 9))
 (segment (start 164.465 125.095) (end 174.625 125.095) (width 0.25) (layer "F.Cu") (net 10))
 (segment (start 172.72 127.635) (end 171.45 126.365) (width 0.25) (layer "F.Cu") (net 11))
 (segment (start 171.45 126.365) (end 167.64 126.365) (width 0.25) (layer "F.Cu") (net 11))
 (segment (start 167.64 126.365) (end 166.37 127.635) (width 0.25) (layer "F.Cu") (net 11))
 (segment (start 166.37 127.635) (end 164.465 127.635) (width 0.25) (layer "F.Cu") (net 11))
 (segment (start 174.625 127.635) (end 172.72 127.635) (width 0.25) (layer "F.Cu") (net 11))
 (segment (start 165.735 130.175) (end 168.275 127.635) (width 0.25) (layer "F.Cu") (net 12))
 (segment (start 168.275 127.635) (end 170.815 127.635) (width 0.25) (layer "F.Cu") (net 12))
 (segment (start 170.815 127.635) (end 173.355 130.175) (width 0.25) (layer "F.Cu") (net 12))
 (segment (start 173.355 130.175) (end 174.625 130.175) (width 0.25) (layer "F.Cu") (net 12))
 (segment (start 164.465 130.175) (end 165.735 130.175) (width 0.25) (layer "F.Cu") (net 12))
 (segment (start 166.37 132.715) (end 169.545 129.54) (width 0.25) (layer "F.Cu") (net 13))
 (segment (start 164.465 132.715) (end 166.37 132.715) (width 0.25) (layer "F.Cu") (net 13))
 (segment (start 165.735 135.255) (end 167.005 136.525) (width 0.25) (layer "F.Cu") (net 14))
 (segment (start 167.005 136.525) (end 172.085 136.525) (width 0.25) (layer "F.Cu") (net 14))
 (segment (start 172.085 136.525) (end 173.355 135.255) (width 0.25) (layer "F.Cu") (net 14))
 (segment (start 173.355 135.255) (end 174.625 135.255) (width 0.25) (layer "F.Cu") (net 14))
 (segment (start 164.465 135.255) (end 165.735 135.255) (width 0.25) (layer "F.Cu") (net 14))
 (segment (start 170.18 132.715) (end 169.545 132.08) (width 0.25) (layer "F.Cu") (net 19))
 (segment (start 174.625 132.715) (end 170.18 132.715) (width 0.25) (layer "F.Cu") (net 19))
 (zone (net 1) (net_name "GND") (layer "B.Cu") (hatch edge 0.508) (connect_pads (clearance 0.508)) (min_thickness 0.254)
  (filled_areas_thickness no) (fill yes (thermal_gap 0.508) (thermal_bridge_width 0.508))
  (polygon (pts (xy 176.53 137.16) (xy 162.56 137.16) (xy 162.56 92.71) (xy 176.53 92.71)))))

